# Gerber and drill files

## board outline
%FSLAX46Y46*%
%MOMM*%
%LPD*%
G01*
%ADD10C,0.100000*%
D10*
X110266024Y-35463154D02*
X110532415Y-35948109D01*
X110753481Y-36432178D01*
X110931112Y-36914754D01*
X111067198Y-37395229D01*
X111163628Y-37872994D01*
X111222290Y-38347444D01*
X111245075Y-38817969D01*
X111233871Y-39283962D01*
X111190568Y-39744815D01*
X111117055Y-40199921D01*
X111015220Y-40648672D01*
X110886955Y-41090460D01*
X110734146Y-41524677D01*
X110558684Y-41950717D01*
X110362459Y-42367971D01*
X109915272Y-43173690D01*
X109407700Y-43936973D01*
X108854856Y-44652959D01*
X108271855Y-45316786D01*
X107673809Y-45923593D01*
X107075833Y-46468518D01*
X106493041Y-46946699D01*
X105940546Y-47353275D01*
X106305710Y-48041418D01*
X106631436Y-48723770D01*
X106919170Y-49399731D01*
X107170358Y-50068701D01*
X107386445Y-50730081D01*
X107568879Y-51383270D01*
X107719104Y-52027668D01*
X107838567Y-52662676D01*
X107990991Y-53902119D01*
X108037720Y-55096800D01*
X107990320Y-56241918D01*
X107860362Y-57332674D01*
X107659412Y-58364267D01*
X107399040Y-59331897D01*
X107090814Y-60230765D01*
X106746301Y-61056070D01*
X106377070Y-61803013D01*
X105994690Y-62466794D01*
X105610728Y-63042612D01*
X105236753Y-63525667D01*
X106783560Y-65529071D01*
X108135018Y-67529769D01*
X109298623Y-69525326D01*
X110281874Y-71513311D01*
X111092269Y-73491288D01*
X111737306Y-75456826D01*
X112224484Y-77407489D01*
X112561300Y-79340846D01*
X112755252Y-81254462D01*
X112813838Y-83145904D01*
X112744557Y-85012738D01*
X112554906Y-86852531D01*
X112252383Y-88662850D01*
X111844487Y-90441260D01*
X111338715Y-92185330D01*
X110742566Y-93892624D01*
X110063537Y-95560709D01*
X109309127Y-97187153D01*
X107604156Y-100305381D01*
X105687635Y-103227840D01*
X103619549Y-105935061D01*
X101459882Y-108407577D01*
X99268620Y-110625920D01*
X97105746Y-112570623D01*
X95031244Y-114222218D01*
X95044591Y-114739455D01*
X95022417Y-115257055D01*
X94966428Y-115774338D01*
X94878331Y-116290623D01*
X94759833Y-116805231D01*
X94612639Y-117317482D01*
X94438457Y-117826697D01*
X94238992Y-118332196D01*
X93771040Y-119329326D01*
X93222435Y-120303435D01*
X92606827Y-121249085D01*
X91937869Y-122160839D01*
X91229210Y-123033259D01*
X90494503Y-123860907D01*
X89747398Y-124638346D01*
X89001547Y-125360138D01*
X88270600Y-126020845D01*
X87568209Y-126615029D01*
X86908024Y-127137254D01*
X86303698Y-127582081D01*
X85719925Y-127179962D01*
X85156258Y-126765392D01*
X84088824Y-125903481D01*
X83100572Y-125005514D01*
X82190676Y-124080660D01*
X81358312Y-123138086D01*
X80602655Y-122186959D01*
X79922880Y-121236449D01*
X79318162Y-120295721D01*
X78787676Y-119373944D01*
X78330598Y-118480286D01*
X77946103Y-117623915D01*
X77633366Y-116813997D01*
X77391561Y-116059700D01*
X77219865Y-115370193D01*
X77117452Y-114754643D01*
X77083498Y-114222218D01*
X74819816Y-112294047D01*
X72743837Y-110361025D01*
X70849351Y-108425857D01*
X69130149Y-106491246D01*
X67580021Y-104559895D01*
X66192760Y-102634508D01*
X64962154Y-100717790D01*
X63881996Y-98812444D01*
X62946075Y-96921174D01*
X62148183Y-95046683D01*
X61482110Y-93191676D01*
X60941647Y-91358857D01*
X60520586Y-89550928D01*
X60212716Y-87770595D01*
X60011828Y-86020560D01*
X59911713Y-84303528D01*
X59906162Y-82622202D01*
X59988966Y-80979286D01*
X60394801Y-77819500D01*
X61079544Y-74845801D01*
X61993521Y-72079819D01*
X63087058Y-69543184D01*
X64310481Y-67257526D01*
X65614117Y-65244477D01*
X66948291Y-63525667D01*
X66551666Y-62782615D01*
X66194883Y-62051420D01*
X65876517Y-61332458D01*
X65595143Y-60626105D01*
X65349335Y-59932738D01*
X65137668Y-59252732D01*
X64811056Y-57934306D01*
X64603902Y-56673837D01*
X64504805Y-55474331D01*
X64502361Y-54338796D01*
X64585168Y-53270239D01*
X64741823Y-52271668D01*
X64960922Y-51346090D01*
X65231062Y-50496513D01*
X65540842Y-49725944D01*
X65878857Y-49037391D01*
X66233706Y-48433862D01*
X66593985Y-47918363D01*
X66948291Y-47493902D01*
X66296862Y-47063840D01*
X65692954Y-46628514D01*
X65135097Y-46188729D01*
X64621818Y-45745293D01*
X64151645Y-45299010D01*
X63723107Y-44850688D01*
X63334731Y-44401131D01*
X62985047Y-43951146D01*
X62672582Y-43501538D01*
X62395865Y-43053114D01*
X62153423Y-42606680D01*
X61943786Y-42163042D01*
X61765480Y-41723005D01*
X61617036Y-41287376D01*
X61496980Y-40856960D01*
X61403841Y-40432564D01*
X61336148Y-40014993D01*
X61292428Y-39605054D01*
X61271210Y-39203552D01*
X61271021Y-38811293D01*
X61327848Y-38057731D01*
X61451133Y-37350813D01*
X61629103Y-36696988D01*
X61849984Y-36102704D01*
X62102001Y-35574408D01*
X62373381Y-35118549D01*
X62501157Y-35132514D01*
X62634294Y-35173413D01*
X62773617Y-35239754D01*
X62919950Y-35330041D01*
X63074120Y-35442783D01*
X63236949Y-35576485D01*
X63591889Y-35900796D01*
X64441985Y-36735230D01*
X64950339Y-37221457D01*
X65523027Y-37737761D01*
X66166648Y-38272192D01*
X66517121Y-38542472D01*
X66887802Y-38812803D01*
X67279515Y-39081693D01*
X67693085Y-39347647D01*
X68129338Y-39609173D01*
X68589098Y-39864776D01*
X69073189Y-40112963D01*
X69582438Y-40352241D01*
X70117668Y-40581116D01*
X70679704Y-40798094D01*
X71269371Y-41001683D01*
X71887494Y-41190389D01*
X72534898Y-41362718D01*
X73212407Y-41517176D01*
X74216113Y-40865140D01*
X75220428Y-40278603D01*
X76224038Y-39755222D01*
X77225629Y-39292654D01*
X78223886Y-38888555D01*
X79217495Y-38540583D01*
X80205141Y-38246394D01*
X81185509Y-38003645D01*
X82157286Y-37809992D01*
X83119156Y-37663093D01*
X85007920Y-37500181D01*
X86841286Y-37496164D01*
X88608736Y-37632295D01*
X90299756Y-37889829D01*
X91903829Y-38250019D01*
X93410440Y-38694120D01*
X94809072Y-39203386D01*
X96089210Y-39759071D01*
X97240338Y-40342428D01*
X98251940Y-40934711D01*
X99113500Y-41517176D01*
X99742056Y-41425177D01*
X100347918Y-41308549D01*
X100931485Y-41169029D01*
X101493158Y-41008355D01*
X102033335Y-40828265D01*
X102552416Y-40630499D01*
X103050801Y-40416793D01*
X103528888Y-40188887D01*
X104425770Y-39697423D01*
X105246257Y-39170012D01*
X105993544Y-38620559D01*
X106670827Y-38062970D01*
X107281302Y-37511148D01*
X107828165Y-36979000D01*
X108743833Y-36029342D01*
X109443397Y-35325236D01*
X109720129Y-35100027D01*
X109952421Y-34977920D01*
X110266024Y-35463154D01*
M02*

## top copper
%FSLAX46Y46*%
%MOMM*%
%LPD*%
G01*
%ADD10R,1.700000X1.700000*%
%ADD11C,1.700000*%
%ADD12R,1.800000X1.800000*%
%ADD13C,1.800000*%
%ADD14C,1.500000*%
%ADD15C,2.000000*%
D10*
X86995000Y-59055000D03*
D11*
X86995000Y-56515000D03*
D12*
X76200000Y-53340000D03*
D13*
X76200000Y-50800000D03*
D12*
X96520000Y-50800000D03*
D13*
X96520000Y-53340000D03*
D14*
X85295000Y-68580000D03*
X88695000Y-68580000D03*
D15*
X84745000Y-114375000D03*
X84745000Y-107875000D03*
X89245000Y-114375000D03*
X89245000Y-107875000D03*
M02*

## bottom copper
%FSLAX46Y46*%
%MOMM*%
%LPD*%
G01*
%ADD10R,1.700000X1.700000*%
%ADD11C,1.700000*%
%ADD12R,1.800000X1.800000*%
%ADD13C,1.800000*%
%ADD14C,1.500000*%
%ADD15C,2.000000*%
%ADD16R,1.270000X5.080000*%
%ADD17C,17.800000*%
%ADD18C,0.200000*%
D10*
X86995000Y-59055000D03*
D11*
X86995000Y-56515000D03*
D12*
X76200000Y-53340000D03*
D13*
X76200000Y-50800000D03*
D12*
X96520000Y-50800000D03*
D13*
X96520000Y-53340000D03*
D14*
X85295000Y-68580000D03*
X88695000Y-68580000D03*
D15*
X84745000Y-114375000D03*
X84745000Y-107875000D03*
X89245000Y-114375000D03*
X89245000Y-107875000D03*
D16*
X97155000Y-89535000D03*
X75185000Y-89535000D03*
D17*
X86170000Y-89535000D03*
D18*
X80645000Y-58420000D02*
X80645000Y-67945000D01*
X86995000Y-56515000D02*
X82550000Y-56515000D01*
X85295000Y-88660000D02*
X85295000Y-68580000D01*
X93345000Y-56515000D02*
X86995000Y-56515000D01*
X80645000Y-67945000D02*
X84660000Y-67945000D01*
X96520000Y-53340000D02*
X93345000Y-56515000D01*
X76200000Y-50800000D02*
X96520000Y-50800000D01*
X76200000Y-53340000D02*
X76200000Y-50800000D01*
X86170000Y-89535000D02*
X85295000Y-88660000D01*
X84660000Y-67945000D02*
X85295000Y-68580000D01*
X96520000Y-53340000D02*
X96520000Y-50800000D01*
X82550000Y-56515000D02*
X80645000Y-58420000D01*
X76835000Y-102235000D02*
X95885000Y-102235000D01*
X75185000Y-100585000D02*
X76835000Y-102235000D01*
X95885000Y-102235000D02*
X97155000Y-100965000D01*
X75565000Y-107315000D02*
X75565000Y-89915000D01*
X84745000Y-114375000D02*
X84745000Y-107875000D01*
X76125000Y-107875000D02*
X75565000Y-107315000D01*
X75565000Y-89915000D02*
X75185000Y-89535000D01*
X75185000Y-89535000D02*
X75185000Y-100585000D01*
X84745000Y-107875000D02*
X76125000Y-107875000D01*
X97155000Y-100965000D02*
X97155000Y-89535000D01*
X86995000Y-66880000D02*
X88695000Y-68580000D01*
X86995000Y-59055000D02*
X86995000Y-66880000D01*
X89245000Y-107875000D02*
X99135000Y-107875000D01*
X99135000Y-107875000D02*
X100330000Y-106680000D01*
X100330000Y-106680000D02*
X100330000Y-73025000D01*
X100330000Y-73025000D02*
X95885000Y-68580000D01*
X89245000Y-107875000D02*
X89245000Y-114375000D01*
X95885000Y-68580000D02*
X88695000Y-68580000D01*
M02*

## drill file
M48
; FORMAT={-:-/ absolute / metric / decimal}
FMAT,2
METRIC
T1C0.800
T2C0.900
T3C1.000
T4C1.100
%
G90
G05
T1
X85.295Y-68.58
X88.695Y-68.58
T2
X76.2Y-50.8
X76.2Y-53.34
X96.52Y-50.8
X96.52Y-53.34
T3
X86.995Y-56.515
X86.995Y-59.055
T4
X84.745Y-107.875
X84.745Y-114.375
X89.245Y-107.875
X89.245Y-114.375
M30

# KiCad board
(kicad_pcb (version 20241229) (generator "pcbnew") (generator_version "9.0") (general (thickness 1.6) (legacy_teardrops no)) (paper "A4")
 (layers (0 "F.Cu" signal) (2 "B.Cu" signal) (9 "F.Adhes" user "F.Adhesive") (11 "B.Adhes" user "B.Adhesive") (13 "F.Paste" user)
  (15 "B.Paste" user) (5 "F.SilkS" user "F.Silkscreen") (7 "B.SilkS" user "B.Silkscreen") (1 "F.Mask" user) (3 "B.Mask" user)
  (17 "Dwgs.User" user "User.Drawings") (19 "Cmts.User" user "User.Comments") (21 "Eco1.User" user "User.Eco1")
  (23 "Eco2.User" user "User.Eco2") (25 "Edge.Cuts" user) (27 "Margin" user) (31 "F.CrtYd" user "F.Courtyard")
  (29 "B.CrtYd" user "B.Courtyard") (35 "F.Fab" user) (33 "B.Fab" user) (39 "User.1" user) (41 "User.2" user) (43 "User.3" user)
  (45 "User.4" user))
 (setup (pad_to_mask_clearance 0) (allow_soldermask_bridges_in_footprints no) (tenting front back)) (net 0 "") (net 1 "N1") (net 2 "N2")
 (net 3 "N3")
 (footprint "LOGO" (layer "F.Cu") (at 86.36 71.12)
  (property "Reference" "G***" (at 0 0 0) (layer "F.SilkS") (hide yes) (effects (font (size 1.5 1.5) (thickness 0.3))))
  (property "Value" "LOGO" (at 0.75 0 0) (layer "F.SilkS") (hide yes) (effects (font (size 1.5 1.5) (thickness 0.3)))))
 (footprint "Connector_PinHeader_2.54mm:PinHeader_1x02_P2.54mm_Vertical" (layer "F.Cu") (at 86.995 59.055 180)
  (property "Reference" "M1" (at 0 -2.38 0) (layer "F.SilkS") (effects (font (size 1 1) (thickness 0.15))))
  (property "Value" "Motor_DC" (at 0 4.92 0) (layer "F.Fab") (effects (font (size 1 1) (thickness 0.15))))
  (pad "1" thru_hole rect (at 0 0 180) (size 1.7 1.7) (drill 1) (layers "*.Cu" "*.Mask") (remove_unused_layers no) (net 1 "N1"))
  (pad "2" thru_hole circle (at 0 2.54 180) (size 1.7 1.7) (drill 1) (layers "*.Cu" "*.Mask") (remove_unused_layers no) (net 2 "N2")))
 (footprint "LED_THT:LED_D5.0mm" (layer "F.Cu") (at 76.2 53.34 90)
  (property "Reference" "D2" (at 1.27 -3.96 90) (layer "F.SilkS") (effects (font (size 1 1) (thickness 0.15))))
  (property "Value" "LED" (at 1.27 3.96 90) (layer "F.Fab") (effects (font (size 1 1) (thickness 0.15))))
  (pad "1" thru_hole rect (at 0 0 90) (size 1.8 1.8) (drill 0.9) (layers "*.Cu" "*.Mask") (remove_unused_layers no) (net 2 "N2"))
  (pad "2" thru_hole circle (at 2.54 0 90) (size 1.8 1.8) (drill 0.9) (layers "*.Cu" "*.Mask") (remove_unused_layers no) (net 2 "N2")))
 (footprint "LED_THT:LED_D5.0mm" (layer "F.Cu") (at 96.52 50.8 -90)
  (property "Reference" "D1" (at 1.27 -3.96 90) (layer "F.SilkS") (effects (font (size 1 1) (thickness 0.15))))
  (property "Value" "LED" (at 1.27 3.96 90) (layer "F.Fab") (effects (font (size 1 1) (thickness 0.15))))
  (pad "1" thru_hole rect (at 0 0 270) (size 1.8 1.8) (drill 0.9) (layers "*.Cu" "*.Mask") (remove_unused_layers no) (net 2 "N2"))
  (pad "2" thru_hole circle (at 2.54 0 270) (size 1.8 1.8) (drill 0.9) (layers "*.Cu" "*.Mask") (remove_unused_layers no) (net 2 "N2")))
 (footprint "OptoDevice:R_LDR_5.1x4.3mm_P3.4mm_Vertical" (layer "F.Cu") (at 85.295 68.58)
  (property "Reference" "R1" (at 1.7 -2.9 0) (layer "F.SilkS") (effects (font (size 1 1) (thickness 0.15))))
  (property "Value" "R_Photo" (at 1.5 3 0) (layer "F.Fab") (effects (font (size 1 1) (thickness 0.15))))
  (pad "1" thru_hole circle (at 0 0) (size 1.5 1.5) (drill 0.8) (layers "*.Cu" "*.Mask") (remove_unused_layers no) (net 2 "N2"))
  (pad "2" thru_hole circle (at 3.4 0) (size 1.5 1.5) (drill 0.8) (layers "*.Cu" "*.Mask") (remove_unused_layers no) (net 1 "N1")))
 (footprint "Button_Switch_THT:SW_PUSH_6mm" (layer "F.Cu") (at 84.745 114.375 90)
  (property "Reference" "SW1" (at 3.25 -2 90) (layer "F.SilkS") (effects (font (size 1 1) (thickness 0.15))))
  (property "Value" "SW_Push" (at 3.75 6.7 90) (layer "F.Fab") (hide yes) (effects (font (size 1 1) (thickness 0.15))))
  (pad "1" thru_hole circle (at 0 0 180) (size 2 2) (drill 1.1) (layers "*.Cu" "*.Mask") (remove_unused_layers no) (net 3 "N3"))
  (pad "1" thru_hole circle (at 6.5 0 180) (size 2 2) (drill 1.1) (layers "*.Cu" "*.Mask") (remove_unused_layers no) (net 3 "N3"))
  (pad "2" thru_hole circle (at 0 4.5 180) (size 2 2) (drill 1.1) (layers "*.Cu" "*.Mask") (remove_unused_layers no) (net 1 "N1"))
  (pad "2" thru_hole circle (at 6.5 4.5 180) (size 2 2) (drill 1.1) (layers "*.Cu" "*.Mask") (remove_unused_layers no) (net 1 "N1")))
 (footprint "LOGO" (layer "B.Cu") (at 86.36 50.8 180)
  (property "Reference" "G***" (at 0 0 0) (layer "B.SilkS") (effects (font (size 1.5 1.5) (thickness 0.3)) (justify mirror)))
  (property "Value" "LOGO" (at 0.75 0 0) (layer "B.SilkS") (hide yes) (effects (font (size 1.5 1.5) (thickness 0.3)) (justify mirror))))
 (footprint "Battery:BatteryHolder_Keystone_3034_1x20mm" (layer "B.Cu") (at 86.17 89.535 180)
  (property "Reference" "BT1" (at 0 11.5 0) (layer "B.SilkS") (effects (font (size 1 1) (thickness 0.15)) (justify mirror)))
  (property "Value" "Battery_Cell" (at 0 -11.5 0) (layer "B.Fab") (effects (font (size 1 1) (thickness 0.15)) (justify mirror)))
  (pad "1" smd rect (at -10.985 0 180) (size 1.27 5.08) (layers "B.Cu" "B.Mask" "B.Paste") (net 3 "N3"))
  (pad "1" smd rect (at 10.985 0 180) (size 1.27 5.08) (layers "B.Cu" "B.Mask" "B.Paste") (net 3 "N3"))
  (pad "2" smd circle (at 0 0 180) (size 17.8 17.8) (layers "B.Cu" "B.Mask") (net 2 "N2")))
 (gr_poly
  (pts (xy 110.266024 35.463154) (xy 110.532415 35.948109) (xy 110.753481 36.432178) (xy 110.931112 36.914754) (xy 111.067198 37.395229)
   (xy 111.163628 37.872994) (xy 111.22229 38.347444) (xy 111.245075 38.817969) (xy 111.233871 39.283962) (xy 111.190568 39.744815)
   (xy 111.117055 40.199921) (xy 111.01522 40.648672) (xy 110.886955 41.09046) (xy 110.734146 41.524677) (xy 110.558684 41.950717)
   (xy 110.362459 42.367971) (xy 109.915272 43.17369) (xy 109.4077 43.936973) (xy 108.854856 44.652959) (xy 108.271855 45.316786)
   (xy 107.673809 45.923593) (xy 107.075833 46.468518) (xy 106.493041 46.946699) (xy 105.940546 47.353275) (xy 106.30571 48.041418)
   (xy 106.631436 48.72377) (xy 106.91917 49.399731) (xy 107.170358 50.068701) (xy 107.386445 50.730081) (xy 107.568879 51.38327)
   (xy 107.719104 52.027668) (xy 107.838567 52.662676) (xy 107.990991 53.902119) (xy 108.03772 55.0968) (xy 107.99032 56.241918)
   (xy 107.860362 57.332674) (xy 107.659412 58.364267) (xy 107.39904 59.331897) (xy 107.090814 60.230765) (xy 106.746301 61.05607)
   (xy 106.37707 61.803013) (xy 105.99469 62.466794) (xy 105.610728 63.042612) (xy 105.236753 63.525667) (xy 106.78356 65.529071)
   (xy 108.135018 67.529769) (xy 109.298623 69.525326) (xy 110.281874 71.513311) (xy 111.092269 73.491288) (xy 111.737306 75.456826)
   (xy 112.224484 77.407489) (xy 112.5613 79.340846) (xy 112.755252 81.254462) (xy 112.813838 83.145904) (xy 112.744557 85.012738)
   (xy 112.554906 86.852531) (xy 112.252383 88.66285) (xy 111.844487 90.44126) (xy 111.338715 92.18533) (xy 110.742566 93.892624)
   (xy 110.063537 95.560709) (xy 109.309127 97.187153) (xy 107.604156 100.305381) (xy 105.687635 103.22784) (xy 103.619549 105.935061)
   (xy 101.459882 108.407577) (xy 99.26862 110.62592) (xy 97.105746 112.570623) (xy 95.031244 114.222218) (xy 95.044591 114.739455)
   (xy 95.022417 115.257055) (xy 94.966428 115.774338) (xy 94.878331 116.290623) (xy 94.759833 116.805231) (xy 94.612639 117.317482)
   (xy 94.438457 117.826697) (xy 94.238992 118.332196) (xy 93.77104 119.329326) (xy 93.222435 120.303435) (xy 92.606827 121.249085)
   (xy 91.937869 122.160839) (xy 91.22921 123.033259) (xy 90.494503 123.860907) (xy 89.747398 124.638346) (xy 89.001547 125.360138)
   (xy 88.2706 126.020845) (xy 87.568209 126.615029) (xy 86.908024 127.137254) (xy 86.303698 127.582081) (xy 85.719925 127.179962)
   (xy 85.156258 126.765392) (xy 84.088824 125.903481) (xy 83.100572 125.005514) (xy 82.190676 124.08066) (xy 81.358312 123.138086)
   (xy 80.602655 122.186959) (xy 79.92288 121.236449) (xy 79.318162 120.295721) (xy 78.787676 119.373944) (xy 78.330598 118.480286)
   (xy 77.946103 117.623915) (xy 77.633366 116.813997) (xy 77.391561 116.0597) (xy 77.219865 115.370193) (xy 77.117452 114.754643)
   (xy 77.083498 114.222218) (xy 74.819816 112.294047) (xy 72.743837 110.361025) (xy 70.849351 108.425857) (xy 69.130149 106.491246)
   (xy 67.580021 104.559895) (xy 66.19276 102.634508) (xy 64.962154 100.71779) (xy 63.881996 98.812444) (xy 62.946075 96.921174)
   (xy 62.148183 95.046683) (xy 61.48211 93.191676) (xy 60.941647 91.358857) (xy 60.520586 89.550928) (xy 60.212716 87.770595)
   (xy 60.011828 86.02056) (xy 59.911713 84.303528) (xy 59.906162 82.622202) (xy 59.988966 80.979286) (xy 60.394801 77.8195)
   (xy 61.079544 74.845801) (xy 61.993521 72.079819) (xy 63.087058 69.543184) (xy 64.310481 67.257526) (xy 65.614117 65.244477)
   (xy 66.948291 63.525667) (xy 66.551666 62.782615) (xy 66.194883 62.05142) (xy 65.876517 61.332458) (xy 65.595143 60.626105)
   (xy 65.349335 59.932738) (xy 65.137668 59.252732) (xy 64.811056 57.934306) (xy 64.603902 56.673837) (xy 64.504805 55.474331)
   (xy 64.502361 54.338796) (xy 64.585168 53.270239) (xy 64.741823 52.271668) (xy 64.960922 51.34609) (xy 65.231062 50.496513)
   (xy 65.540842 49.725944) (xy 65.878857 49.037391) (xy 66.233706 48.433862) (xy 66.593985 47.918363) (xy 66.948291 47.493902)
   (xy 66.296862 47.06384) (xy 65.692954 46.628514) (xy 65.135097 46.188729) (xy 64.621818 45.745293) (xy 64.151645 45.29901)
   (xy 63.723107 44.850688) (xy 63.334731 44.401131) (xy 62.985047 43.951146) (xy 62.672582 43.501538) (xy 62.395865 43.053114)
   (xy 62.153423 42.60668) (xy 61.943786 42.163042) (xy 61.76548 41.723005) (xy 61.617036 41.287376) (xy 61.49698 40.85696)
   (xy 61.403841 40.432564) (xy 61.336148 40.014993) (xy 61.292428 39.605054) (xy 61.27121 39.203552) (xy 61.271021 38.811293)
   (xy 61.327848 38.057731) (xy 61.451133 37.350813) (xy 61.629103 36.696988) (xy 61.849984 36.102704) (xy 62.102001 35.574408)
   (xy 62.373381 35.118549) (xy 62.501157 35.132514) (xy 62.634294 35.173413) (xy 62.773617 35.239754) (xy 62.91995 35.330041)
   (xy 63.07412 35.442783) (xy 63.236949 35.576485) (xy 63.591889 35.900796) (xy 64.441985 36.73523) (xy 64.950339 37.221457)
   (xy 65.523027 37.737761) (xy 66.166648 38.272192) (xy 66.517121 38.542472) (xy 66.887802 38.812803) (xy 67.279515 39.081693)
   (xy 67.693085 39.347647) (xy 68.129338 39.609173) (xy 68.589098 39.864776) (xy 69.073189 40.112963) (xy 69.582438 40.352241)
   (xy 70.117668 40.581116) (xy 70.679704 40.798094) (xy 71.269371 41.001683) (xy 71.887494 41.190389) (xy 72.534898 41.362718)
   (xy 73.212407 41.517176) (xy 74.216113 40.86514) (xy 75.220428 40.278603) (xy 76.224038 39.755222) (xy 77.225629 39.292654)
   (xy 78.223886 38.888555) (xy 79.217495 38.540583) (xy 80.205141 38.246394) (xy 81.185509 38.003645) (xy 82.157286 37.809992)
   (xy 83.119156 37.663093) (xy 85.00792 37.500181) (xy 86.841286 37.496164) (xy 88.608736 37.632295) (xy 90.299756 37.889829)
   (xy 91.903829 38.250019) (xy 93.41044 38.69412) (xy 94.809072 39.203386) (xy 96.08921 39.759071) (xy 97.240338 40.342428)
   (xy 98.25194 40.934711) (xy 99.1135 41.517176) (xy 99.742056 41.425177) (xy 100.347918 41.308549) (xy 100.931485 41.169029)
   (xy 101.493158 41.008355) (xy 102.033335 40.828265) (xy 102.552416 40.630499) (xy 103.050801 40.416793) (xy 103.528888 40.188887)
   (xy 104.42577 39.697423) (xy 105.246257 39.170012) (xy 105.993544 38.620559) (xy 106.670827 38.06297) (xy 107.281302 37.511148)
   (xy 107.828165 36.979) (xy 108.743833 36.029342) (xy 109.443397 35.325236) (xy 109.720129 35.100027) (xy 109.952421 34.97792))
  (stroke (width 0.1) (type solid)) (fill no) (layer "Edge.Cuts"))
 (segment (start 80.645 58.42) (end 80.645 67.945) (width 0.2) (layer "B.Cu") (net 2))
 (segment (start 86.995 56.515) (end 82.55 56.515) (width 0.2) (layer "B.Cu") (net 2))
 (segment (start 85.295 88.66) (end 85.295 68.58) (width 0.2) (layer "B.Cu") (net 2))
 (segment (start 93.345 56.515) (end 86.995 56.515) (width 0.2) (layer "B.Cu") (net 2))
 (segment (start 80.645 67.945) (end 84.66 67.945) (width 0.2) (layer "B.Cu") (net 2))
 (segment (start 96.52 53.34) (end 93.345 56.515) (width 0.2) (layer "B.Cu") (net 2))
 (segment (start 76.2 50.8) (end 96.52 50.8) (width 0.2) (layer "B.Cu") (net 2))
 (segment (start 76.2 53.34) (end 76.2 50.8) (width 0.2) (layer "B.Cu") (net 2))
 (segment (start 86.17 89.535) (end 85.295 88.66) (width 0.2) (layer "B.Cu") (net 2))
 (segment (start 84.66 67.945) (end 85.295 68.58) (width 0.2) (layer "B.Cu") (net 2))
 (segment (start 96.52 53.34) (end 96.52 50.8) (width 0.2) (layer "B.Cu") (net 2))
 (segment (start 82.55 56.515) (end 80.645 58.42) (width 0.2) (layer "B.Cu") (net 2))
 (segment (start 76.835 102.235) (end 95.885 102.235) (width 0.2) (layer "B.Cu") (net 3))
 (segment (start 75.185 100.585) (end 76.835 102.235) (width 0.2) (layer "B.Cu") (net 3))
 (segment (start 95.885 102.235) (end 97.155 100.965) (width 0.2) (layer "B.Cu") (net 3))
 (segment (start 75.565 107.315) (end 75.565 89.915) (width 0.2) (layer "B.Cu") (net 3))
 (segment (start 84.745 114.375) (end 84.745 107.875) (width 0.2) (layer "B.Cu") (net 3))
 (segment (start 76.125 107.875) (end 75.565 107.315) (width 0.2) (layer "B.Cu") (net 3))
 (segment (start 75.565 89.915) (end 75.185 89.535) (width 0.2) (layer "B.Cu") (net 3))
 (segment (start 75.185 89.535) (end 75.185 100.585) (width 0.2) (layer "B.Cu") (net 3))
 (segment (start 84.745 107.875) (end 76.125 107.875) (width 0.2) (layer "B.Cu") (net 3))
 (segment (start 97.155 100.965) (end 97.155 89.535) (width 0.2) (layer "B.Cu") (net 3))
 (segment (start 86.995 66.88) (end 88.695 68.58) (width 0.2) (layer "B.Cu") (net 1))
 (segment (start 86.995 59.055) (end 86.995 66.88) (width 0.2) (layer "B.Cu") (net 1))
 (segment (start 89.245 107.875) (end 99.135 107.875) (width 0.2) (layer "B.Cu") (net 1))
 (segment (start 99.135 107.875) (end 100.33 106.68) (width 0.2) (layer "B.Cu") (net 1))
 (segment (start 100.33 106.68) (end 100.33 73.025) (width 0.2) (layer "B.Cu") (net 1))
 (segment (start 100.33 73.025) (end 95.885 68.58) (width 0.2) (layer "B.Cu") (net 1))
 (segment (start 89.245 107.875) (end 89.245 114.375) (width 0.2) (layer "B.Cu") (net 1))
 (segment (start 95.885 68.58) (end 88.695 68.58) (width 0.2) (layer "B.Cu") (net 1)))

